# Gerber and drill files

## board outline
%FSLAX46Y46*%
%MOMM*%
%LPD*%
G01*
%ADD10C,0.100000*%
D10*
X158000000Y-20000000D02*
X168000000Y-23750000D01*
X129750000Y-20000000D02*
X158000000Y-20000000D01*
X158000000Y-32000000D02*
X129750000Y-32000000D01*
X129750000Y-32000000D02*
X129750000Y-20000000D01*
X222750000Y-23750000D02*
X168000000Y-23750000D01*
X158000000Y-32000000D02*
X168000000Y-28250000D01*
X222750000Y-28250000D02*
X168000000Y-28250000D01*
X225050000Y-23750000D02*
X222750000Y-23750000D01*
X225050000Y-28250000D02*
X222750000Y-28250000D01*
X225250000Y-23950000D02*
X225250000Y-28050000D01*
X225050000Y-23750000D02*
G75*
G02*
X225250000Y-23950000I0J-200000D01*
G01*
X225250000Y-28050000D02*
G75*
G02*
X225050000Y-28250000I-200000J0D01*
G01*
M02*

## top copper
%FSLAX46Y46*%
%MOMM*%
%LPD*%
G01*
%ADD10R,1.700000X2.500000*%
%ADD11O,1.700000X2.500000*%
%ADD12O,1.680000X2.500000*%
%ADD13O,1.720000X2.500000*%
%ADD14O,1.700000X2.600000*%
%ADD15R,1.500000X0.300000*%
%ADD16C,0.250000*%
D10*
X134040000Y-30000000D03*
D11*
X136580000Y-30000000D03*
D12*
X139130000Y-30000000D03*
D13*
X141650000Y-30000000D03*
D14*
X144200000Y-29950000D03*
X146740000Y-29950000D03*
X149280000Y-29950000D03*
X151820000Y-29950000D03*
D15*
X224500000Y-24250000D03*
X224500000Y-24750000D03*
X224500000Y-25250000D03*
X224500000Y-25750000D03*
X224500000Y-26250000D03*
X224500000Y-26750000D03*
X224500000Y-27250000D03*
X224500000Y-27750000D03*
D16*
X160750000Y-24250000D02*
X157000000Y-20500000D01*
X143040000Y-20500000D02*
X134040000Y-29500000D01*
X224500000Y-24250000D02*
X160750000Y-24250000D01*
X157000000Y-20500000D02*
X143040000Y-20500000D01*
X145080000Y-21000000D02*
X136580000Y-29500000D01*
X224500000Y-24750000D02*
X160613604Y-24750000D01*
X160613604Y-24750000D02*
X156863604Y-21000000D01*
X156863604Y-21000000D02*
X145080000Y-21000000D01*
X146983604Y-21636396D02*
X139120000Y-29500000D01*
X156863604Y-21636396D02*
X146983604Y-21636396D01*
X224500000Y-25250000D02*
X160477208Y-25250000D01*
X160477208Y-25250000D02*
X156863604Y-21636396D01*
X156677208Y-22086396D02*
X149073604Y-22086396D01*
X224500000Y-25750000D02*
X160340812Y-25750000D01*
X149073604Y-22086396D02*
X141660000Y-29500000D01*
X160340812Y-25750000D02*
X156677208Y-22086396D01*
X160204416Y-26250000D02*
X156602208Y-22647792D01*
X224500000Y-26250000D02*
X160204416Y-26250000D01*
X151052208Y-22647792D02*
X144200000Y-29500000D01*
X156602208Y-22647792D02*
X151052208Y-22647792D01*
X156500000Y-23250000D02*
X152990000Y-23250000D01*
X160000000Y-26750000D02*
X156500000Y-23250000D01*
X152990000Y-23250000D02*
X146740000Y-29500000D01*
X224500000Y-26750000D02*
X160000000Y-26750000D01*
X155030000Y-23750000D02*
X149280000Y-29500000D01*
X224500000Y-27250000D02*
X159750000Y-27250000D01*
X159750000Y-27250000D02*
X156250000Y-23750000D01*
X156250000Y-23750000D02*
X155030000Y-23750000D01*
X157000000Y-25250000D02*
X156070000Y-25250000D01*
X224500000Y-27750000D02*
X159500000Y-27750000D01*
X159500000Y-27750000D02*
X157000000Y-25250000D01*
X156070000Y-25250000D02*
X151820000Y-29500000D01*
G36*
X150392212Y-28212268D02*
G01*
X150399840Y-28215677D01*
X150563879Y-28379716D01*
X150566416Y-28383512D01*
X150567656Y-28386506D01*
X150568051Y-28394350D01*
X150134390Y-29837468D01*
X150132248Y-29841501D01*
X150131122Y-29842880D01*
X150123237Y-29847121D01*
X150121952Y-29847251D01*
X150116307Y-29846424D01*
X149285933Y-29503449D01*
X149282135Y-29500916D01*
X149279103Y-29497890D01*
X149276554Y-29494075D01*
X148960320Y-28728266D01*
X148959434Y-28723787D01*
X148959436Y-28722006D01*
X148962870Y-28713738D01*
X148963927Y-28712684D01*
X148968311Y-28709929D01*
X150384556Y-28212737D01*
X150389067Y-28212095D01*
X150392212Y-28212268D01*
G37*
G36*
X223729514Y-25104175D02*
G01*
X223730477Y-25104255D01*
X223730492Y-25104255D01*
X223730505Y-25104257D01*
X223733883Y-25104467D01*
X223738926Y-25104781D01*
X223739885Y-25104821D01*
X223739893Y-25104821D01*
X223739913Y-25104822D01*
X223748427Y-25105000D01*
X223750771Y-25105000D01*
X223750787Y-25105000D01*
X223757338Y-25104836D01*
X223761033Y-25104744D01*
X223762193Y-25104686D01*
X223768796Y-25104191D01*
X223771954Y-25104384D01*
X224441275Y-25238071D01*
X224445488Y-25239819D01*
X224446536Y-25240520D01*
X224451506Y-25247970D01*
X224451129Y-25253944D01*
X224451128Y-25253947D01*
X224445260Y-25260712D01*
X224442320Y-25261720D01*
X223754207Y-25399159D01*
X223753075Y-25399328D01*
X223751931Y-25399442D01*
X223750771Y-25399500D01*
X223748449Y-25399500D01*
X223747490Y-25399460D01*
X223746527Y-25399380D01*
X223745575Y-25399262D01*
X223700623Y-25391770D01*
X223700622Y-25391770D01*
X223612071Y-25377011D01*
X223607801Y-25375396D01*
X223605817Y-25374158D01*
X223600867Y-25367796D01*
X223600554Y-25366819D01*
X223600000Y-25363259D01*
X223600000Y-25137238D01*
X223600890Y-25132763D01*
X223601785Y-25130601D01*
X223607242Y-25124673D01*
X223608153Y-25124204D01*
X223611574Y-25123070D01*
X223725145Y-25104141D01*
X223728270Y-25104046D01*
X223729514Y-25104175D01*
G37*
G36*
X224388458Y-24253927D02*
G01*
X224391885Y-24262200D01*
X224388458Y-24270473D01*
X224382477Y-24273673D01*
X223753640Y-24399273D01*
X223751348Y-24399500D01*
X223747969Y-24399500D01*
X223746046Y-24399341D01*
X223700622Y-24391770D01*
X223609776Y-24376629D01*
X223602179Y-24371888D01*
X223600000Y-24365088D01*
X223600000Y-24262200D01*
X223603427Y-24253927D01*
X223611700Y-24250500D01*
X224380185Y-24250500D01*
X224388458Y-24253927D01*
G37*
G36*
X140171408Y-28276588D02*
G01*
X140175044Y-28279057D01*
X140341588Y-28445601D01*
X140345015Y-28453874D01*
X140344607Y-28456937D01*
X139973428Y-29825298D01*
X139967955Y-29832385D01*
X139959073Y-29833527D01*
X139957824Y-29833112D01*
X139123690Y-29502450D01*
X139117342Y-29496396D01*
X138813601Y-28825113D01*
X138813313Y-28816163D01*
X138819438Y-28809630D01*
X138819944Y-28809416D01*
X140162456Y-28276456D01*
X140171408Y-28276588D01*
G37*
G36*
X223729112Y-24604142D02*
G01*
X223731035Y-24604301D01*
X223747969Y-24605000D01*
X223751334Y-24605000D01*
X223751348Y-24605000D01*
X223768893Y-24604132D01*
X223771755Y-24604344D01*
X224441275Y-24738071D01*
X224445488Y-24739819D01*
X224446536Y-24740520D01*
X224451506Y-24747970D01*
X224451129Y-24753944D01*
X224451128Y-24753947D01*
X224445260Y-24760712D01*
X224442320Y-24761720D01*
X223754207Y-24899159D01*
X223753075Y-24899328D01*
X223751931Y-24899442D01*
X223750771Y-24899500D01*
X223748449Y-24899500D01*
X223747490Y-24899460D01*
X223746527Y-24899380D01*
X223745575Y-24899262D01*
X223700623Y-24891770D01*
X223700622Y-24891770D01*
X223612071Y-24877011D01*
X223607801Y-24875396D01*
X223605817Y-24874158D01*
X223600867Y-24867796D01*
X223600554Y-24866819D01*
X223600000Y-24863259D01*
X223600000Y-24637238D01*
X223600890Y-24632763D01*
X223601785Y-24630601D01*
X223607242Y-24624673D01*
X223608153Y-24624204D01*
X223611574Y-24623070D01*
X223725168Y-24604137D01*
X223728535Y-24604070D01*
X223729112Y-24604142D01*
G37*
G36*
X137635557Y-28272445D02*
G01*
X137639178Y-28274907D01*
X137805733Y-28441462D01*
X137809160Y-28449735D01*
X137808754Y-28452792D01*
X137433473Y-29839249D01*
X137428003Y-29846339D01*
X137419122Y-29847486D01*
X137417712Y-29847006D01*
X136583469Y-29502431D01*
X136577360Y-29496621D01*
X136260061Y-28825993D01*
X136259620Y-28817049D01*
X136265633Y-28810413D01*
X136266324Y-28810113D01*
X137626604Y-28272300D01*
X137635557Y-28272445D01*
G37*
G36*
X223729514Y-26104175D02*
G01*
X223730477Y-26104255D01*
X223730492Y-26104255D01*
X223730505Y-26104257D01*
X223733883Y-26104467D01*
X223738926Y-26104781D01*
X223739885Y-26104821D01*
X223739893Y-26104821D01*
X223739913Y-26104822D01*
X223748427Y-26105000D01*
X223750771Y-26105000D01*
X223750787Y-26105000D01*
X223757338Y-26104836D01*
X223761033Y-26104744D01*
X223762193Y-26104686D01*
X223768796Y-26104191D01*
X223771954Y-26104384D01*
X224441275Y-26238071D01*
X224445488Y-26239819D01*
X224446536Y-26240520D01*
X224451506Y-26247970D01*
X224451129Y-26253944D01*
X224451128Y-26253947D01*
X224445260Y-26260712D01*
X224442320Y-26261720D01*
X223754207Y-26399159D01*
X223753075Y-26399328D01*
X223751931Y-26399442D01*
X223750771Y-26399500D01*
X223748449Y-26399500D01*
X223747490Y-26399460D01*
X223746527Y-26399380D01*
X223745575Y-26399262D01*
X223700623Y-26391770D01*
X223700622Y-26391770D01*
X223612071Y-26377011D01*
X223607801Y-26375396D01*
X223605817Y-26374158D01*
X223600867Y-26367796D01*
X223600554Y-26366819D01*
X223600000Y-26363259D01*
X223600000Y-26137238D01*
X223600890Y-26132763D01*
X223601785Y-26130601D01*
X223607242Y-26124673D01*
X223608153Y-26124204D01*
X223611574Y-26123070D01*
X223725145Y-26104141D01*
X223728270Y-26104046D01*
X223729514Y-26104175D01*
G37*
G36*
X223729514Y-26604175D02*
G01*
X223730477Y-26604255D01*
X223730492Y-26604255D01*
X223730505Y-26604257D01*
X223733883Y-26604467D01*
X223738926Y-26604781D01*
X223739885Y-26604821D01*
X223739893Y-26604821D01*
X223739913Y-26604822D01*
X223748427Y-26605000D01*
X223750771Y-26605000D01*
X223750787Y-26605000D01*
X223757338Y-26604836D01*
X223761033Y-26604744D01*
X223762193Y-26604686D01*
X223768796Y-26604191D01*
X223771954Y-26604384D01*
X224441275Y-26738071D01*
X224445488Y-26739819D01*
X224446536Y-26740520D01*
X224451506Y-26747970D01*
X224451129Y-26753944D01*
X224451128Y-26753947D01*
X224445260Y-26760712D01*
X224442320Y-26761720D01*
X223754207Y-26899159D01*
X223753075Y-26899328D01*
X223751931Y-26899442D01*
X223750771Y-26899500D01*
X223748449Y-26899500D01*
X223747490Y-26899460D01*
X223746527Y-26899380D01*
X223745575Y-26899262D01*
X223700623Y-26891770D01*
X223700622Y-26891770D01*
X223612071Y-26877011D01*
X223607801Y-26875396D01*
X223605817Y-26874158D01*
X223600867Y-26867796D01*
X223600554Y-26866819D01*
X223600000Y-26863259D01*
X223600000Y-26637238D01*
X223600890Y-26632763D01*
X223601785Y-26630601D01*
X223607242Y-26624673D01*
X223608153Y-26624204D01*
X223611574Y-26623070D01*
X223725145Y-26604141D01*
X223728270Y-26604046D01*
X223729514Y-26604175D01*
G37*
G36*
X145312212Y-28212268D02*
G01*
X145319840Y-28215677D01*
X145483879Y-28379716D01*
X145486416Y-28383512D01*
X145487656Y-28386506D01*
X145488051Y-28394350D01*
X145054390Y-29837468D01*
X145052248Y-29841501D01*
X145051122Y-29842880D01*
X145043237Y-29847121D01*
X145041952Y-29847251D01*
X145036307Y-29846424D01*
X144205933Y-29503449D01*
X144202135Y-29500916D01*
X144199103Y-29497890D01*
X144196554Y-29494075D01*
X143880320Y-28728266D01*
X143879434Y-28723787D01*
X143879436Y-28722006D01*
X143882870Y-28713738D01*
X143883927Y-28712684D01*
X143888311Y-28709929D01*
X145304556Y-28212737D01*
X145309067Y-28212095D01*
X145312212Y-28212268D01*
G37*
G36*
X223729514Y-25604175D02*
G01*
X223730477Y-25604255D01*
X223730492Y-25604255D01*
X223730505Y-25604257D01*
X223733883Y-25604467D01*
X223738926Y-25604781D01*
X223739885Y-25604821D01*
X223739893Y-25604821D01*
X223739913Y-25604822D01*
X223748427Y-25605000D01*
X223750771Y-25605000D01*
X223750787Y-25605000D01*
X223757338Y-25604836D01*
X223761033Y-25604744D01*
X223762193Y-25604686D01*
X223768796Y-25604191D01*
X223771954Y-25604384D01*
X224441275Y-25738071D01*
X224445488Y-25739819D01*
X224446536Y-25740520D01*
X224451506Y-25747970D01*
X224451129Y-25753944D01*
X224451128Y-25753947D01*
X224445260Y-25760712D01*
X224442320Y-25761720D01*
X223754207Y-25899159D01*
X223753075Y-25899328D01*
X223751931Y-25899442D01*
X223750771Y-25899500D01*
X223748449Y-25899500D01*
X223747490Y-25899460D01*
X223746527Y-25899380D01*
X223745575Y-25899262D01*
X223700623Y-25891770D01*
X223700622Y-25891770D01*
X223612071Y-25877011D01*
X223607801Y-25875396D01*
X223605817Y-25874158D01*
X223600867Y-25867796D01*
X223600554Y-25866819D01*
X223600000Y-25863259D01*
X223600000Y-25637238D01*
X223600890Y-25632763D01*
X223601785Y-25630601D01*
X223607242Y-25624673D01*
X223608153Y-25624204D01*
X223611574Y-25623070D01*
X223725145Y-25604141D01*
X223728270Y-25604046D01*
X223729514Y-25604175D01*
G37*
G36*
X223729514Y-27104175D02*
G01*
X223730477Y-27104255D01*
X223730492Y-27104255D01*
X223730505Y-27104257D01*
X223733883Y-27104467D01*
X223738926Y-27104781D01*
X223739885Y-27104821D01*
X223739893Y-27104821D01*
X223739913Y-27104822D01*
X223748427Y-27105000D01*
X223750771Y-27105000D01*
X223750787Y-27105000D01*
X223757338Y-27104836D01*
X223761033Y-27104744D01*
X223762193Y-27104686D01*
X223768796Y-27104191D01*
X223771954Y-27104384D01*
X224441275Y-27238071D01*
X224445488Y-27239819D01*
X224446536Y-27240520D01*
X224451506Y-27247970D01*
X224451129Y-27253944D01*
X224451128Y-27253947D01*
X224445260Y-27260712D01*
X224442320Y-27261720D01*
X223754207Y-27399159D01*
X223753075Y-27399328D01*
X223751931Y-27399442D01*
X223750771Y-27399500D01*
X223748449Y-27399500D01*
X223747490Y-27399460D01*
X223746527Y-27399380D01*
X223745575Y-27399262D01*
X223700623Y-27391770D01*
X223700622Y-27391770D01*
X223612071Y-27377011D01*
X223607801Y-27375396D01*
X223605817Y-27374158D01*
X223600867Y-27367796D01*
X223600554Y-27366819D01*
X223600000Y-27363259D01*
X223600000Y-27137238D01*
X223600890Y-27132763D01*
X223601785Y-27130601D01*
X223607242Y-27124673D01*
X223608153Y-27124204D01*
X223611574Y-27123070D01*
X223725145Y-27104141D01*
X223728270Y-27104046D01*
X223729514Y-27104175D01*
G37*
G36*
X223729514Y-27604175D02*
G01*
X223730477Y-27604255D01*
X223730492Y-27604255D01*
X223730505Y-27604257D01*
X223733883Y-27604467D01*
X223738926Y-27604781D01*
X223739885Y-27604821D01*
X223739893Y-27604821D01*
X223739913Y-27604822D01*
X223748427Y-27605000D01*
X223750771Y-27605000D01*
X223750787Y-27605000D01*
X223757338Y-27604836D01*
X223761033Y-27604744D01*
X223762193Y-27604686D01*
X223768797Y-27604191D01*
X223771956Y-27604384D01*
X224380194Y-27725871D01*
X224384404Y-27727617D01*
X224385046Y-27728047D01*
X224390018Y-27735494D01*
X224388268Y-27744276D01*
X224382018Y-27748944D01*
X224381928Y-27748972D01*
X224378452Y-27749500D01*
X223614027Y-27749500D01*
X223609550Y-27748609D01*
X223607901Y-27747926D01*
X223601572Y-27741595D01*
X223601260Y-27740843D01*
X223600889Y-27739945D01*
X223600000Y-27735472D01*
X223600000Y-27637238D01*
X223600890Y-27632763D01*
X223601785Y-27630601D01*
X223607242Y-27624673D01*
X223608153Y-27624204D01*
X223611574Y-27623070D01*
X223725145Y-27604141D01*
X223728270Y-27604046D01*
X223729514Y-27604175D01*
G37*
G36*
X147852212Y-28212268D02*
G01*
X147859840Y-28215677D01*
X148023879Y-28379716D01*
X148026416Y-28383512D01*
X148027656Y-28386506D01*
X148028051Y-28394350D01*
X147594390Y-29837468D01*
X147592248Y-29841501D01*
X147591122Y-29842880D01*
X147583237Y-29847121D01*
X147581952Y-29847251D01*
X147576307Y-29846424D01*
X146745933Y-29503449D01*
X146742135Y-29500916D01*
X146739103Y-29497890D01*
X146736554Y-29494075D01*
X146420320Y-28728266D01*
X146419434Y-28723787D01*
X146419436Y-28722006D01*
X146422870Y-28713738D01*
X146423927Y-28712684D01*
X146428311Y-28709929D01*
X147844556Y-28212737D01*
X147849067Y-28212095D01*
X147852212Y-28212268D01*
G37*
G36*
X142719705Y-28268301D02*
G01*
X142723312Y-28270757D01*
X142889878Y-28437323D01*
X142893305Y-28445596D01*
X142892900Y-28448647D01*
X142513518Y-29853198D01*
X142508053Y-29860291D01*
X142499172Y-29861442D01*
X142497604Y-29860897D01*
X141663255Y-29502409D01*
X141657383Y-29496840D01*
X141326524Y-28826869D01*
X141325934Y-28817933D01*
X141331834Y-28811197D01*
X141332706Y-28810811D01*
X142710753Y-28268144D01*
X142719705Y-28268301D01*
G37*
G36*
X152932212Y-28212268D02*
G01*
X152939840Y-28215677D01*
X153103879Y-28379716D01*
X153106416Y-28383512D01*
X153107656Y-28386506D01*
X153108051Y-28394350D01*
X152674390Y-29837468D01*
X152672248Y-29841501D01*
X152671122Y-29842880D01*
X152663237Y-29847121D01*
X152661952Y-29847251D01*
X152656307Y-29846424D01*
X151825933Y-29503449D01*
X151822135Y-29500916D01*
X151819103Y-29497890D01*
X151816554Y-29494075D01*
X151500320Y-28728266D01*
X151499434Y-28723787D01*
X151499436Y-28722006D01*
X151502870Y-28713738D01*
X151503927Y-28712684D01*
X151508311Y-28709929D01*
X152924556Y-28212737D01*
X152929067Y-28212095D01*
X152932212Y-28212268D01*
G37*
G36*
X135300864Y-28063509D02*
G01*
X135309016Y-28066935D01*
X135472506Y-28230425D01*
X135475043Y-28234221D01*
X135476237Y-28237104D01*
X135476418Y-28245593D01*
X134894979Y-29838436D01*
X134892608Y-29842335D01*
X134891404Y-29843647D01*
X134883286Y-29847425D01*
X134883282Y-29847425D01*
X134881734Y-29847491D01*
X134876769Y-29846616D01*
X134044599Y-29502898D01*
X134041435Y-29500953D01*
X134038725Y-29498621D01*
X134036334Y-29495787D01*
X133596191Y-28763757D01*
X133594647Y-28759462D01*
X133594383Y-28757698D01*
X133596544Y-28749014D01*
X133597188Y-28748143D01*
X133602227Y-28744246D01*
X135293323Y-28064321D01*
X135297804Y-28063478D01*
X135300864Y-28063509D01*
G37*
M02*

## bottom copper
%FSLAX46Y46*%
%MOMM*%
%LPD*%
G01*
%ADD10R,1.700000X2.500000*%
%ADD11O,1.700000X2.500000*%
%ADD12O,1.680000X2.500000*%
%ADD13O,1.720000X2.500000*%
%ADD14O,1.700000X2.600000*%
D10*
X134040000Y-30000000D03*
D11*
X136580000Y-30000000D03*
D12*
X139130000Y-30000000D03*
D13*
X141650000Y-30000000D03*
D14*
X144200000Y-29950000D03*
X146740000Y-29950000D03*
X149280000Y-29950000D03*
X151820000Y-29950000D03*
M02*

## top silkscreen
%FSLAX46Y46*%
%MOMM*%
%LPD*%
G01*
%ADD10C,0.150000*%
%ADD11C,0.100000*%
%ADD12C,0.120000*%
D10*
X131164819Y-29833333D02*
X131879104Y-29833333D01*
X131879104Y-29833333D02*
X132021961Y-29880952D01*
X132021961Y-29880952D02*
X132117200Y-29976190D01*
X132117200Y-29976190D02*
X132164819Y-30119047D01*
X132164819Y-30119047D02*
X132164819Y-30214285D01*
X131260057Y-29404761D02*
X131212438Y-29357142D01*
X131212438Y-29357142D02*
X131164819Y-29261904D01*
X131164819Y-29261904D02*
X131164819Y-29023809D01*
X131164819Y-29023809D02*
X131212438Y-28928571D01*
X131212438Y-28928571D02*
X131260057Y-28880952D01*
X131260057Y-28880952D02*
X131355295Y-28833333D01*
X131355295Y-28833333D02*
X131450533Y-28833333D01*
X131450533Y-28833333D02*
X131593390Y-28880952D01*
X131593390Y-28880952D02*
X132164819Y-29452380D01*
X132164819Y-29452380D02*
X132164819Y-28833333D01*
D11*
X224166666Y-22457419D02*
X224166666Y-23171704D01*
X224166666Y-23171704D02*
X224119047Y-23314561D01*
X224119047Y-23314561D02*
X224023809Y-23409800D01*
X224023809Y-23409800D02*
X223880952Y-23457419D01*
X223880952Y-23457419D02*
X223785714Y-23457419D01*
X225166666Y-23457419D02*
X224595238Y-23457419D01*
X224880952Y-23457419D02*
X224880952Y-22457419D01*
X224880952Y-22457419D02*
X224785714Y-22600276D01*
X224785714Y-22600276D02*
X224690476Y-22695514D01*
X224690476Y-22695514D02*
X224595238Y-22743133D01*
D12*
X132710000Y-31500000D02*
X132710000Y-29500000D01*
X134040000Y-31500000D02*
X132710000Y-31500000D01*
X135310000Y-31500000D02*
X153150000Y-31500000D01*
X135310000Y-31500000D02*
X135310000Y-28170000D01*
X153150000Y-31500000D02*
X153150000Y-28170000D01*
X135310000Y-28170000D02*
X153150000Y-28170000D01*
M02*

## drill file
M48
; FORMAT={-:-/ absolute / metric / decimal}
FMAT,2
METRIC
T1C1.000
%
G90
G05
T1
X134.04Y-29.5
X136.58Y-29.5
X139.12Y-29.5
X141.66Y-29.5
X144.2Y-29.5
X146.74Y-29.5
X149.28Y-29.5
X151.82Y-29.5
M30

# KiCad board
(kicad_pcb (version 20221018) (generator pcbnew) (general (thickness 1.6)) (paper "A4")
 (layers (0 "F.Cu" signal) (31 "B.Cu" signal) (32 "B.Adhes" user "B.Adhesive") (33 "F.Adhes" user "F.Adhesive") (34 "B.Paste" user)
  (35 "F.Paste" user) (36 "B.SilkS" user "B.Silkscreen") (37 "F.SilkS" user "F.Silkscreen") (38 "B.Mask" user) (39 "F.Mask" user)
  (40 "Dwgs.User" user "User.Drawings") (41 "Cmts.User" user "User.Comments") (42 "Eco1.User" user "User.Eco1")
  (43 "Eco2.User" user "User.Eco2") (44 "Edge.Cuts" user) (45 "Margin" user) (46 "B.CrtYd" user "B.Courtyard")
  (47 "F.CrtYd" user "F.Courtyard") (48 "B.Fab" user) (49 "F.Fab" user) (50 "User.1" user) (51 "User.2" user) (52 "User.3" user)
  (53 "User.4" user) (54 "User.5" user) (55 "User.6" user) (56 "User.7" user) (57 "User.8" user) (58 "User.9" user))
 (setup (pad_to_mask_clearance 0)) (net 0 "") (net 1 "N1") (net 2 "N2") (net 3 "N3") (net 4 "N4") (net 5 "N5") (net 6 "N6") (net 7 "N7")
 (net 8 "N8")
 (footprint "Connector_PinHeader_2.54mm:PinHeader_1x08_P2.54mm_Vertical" (layer "F.Cu") (at 134.04 29.5 90)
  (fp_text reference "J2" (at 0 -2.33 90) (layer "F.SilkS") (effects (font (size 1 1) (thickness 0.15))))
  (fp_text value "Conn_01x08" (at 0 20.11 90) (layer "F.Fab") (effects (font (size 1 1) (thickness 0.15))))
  (fp_line (start -2 -1.33) (end 0 -1.33) (stroke (width 0.12) (type solid)) (layer "F.SilkS"))
  (fp_line (start -2 0) (end -2 -1.33) (stroke (width 0.12) (type solid)) (layer "F.SilkS"))
  (fp_line (start -2 1.27) (end -2 19.11) (stroke (width 0.12) (type solid)) (layer "F.SilkS"))
  (fp_line (start -2 1.27) (end 1.33 1.27) (stroke (width 0.12) (type solid)) (layer "F.SilkS"))
  (fp_line (start -2 19.11) (end 1.33 19.11) (stroke (width 0.12) (type solid)) (layer "F.SilkS"))
  (fp_line (start 1.33 1.27) (end 1.33 19.11) (stroke (width 0.12) (type solid)) (layer "F.SilkS"))
  (pad "1" thru_hole rect (at 0 0 90) (size 2.5 1.7) (drill 1 (offset -0.5 0)) (layers "*.Cu" "*.Mask") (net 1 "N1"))
  (pad "2" thru_hole oval (at 0 2.54 90) (size 2.5 1.7) (drill 1 (offset -0.5 0)) (layers "*.Cu" "*.Mask") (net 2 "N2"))
  (pad "3" thru_hole oval (at 0 5.08 90) (size 2.5 1.68) (drill 1 (offset -0.5 0.01)) (layers "*.Cu" "*.Mask") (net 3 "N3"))
  (pad "4" thru_hole oval (at 0 7.62 90) (size 2.5 1.72) (drill 1 (offset -0.5 -0.01)) (layers "*.Cu" "*.Mask") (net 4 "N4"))
  (pad "5" thru_hole oval (at 0 10.16 90) (size 2.6 1.7) (drill 1 (offset -0.45 0)) (layers "*.Cu" "*.Mask") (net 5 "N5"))
  (pad "6" thru_hole oval (at 0 12.7 90) (size 2.6 1.7) (drill 1 (offset -0.45 0)) (layers "*.Cu" "*.Mask") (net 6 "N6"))
  (pad "7" thru_hole oval (at 0 15.24 90) (size 2.6 1.7) (drill 1 (offset -0.45 0)) (layers "*.Cu" "*.Mask") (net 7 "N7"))
  (pad "8" thru_hole oval (at 0 17.78 90) (size 2.6 1.7) (drill 1 (offset -0.45 0)) (layers "*.Cu" "*.Mask") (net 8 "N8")))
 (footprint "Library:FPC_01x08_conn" (layer "F.Cu") (at 224.5 26)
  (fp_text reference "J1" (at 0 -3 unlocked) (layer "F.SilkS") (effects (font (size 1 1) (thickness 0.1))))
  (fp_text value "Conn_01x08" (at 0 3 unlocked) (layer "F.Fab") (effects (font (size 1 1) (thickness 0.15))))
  (fp_line (start 0.55 -2.25) (end -1.75 -2.25) (stroke (width 0.1) (type default)) (layer "Edge.Cuts"))
  (fp_line (start 0.55 2.25) (end -1.75 2.25) (stroke (width 0.1) (type default)) (layer "Edge.Cuts"))
  (fp_line (start 0.75 -2.05) (end 0.75 2.05) (stroke (width 0.1) (type default)) (layer "Edge.Cuts"))
  (fp_arc (start 0.55 -2.25) (mid 0.691422 -2.191422) (end 0.75 -2.05) (stroke (width 0.1) (type default)) (layer "Edge.Cuts"))
  (fp_arc (start 0.75 2.05) (mid 0.691422 2.191422) (end 0.55 2.25) (stroke (width 0.1) (type default)) (layer "Edge.Cuts"))
  (pad "1" smd rect (at 0 -1.75) (size 1.5 0.3) (layers "F.Cu" "F.Paste" "F.Mask") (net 1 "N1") (thermal_bridge_angle 45))
  (pad "2" smd rect (at 0 -1.25) (size 1.5 0.3) (layers "F.Cu" "F.Paste" "F.Mask") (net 2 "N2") (thermal_bridge_angle 45))
  (pad "3" smd rect (at 0 -0.75) (size 1.5 0.3) (layers "F.Cu" "F.Paste" "F.Mask") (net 3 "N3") (thermal_bridge_angle 45))
  (pad "4" smd rect (at 0 -0.25) (size 1.5 0.3) (layers "F.Cu" "F.Paste" "F.Mask") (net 4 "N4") (thermal_bridge_angle 45))
  (pad "5" smd rect (at 0 0.25) (size 1.5 0.3) (layers "F.Cu" "F.Paste" "F.Mask") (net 5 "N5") (thermal_bridge_angle 45))
  (pad "6" smd rect (at 0 0.75) (size 1.5 0.3) (layers "F.Cu" "F.Paste" "F.Mask") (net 6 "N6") (thermal_bridge_angle 45))
  (pad "7" smd rect (at 0 1.25) (size 1.5 0.3) (layers "F.Cu" "F.Paste" "F.Mask") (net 7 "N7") (thermal_bridge_angle 45))
  (pad "8" smd rect (at 0 1.75) (size 1.5 0.3) (layers "F.Cu" "F.Paste" "F.Mask") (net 8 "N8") (thermal_bridge_angle 45)))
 (gr_line (start 158 20) (end 168 23.75) (stroke (width 0.1) (type default)) (layer "Edge.Cuts"))
 (gr_line (start 129.75 20) (end 158 20) (stroke (width 0.1) (type default)) (layer "Edge.Cuts"))
 (gr_line (start 158 32) (end 129.75 32) (stroke (width 0.1) (type default)) (layer "Edge.Cuts"))
 (gr_line (start 129.75 32) (end 129.75 20) (stroke (width 0.1) (type default)) (layer "Edge.Cuts"))
 (gr_line (start 222.75 23.75) (end 168 23.75) (stroke (width 0.1) (type default)) (layer "Edge.Cuts"))
 (gr_line (start 158 32) (end 168 28.25) (stroke (width 0.1) (type default)) (layer "Edge.Cuts"))
 (gr_line (start 222.75 28.25) (end 168 28.25) (stroke (width 0.1) (type default)) (layer "Edge.Cuts"))
 (segment (start 160.75 24.25) (end 157 20.5) (width 0.25) (layer "F.Cu") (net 1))
 (segment (start 143.04 20.5) (end 134.04 29.5) (width 0.25) (layer "F.Cu") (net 1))
 (segment (start 224.5 24.25) (end 160.75 24.25) (width 0.25) (layer "F.Cu") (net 1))
 (segment (start 157 20.5) (end 143.04 20.5) (width 0.25) (layer "F.Cu") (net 1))
 (segment (start 145.08 21) (end 136.58 29.5) (width 0.25) (layer "F.Cu") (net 2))
 (segment (start 224.5 24.75) (end 160.613604 24.75) (width 0.25) (layer "F.Cu") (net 2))
 (segment (start 160.613604 24.75) (end 156.863604 21) (width 0.25) (layer "F.Cu") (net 2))
 (segment (start 156.863604 21) (end 145.08 21) (width 0.25) (layer "F.Cu") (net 2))
 (segment (start 146.983604 21.636396) (end 139.12 29.5) (width 0.25) (layer "F.Cu") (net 3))
 (segment (start 156.863604 21.636396) (end 146.983604 21.636396) (width 0.25) (layer "F.Cu") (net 3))
 (segment (start 224.5 25.25) (end 160.477208 25.25) (width 0.25) (layer "F.Cu") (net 3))
 (segment (start 160.477208 25.25) (end 156.863604 21.636396) (width 0.25) (layer "F.Cu") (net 3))
 (segment (start 156.677208 22.086396) (end 149.073604 22.086396) (width 0.25) (layer "F.Cu") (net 4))
 (segment (start 224.5 25.75) (end 160.340812 25.75) (width 0.25) (layer "F.Cu") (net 4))
 (segment (start 149.073604 22.086396) (end 141.66 29.5) (width 0.25) (layer "F.Cu") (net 4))
 (segment (start 160.340812 25.75) (end 156.677208 22.086396) (width 0.25) (layer "F.Cu") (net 4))
 (segment (start 160.204416 26.25) (end 156.602208 22.647792) (width 0.25) (layer "F.Cu") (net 5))
 (segment (start 224.5 26.25) (end 160.204416 26.25) (width 0.25) (layer "F.Cu") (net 5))
 (segment (start 151.052208 22.647792) (end 144.2 29.5) (width 0.25) (layer "F.Cu") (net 5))
 (segment (start 156.602208 22.647792) (end 151.052208 22.647792) (width 0.25) (layer "F.Cu") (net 5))
 (segment (start 156.5 23.25) (end 152.99 23.25) (width 0.25) (layer "F.Cu") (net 6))
 (segment (start 160 26.75) (end 156.5 23.25) (width 0.25) (layer "F.Cu") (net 6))
 (segment (start 152.99 23.25) (end 146.74 29.5) (width 0.25) (layer "F.Cu") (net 6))
 (segment (start 224.5 26.75) (end 160 26.75) (width 0.25) (layer "F.Cu") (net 6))
 (segment (start 155.03 23.75) (end 149.28 29.5) (width 0.25) (layer "F.Cu") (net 7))
 (segment (start 224.5 27.25) (end 159.75 27.25) (width 0.25) (layer "F.Cu") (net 7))
 (segment (start 159.75 27.25) (end 156.25 23.75) (width 0.25) (layer "F.Cu") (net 7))
 (segment (start 156.25 23.75) (end 155.03 23.75) (width 0.25) (layer "F.Cu") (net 7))
 (segment (start 157 25.25) (end 156.07 25.25) (width 0.25) (layer "F.Cu") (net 8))
 (segment (start 224.5 27.75) (end 159.5 27.75) (width 0.25) (layer "F.Cu") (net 8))
 (segment (start 159.5 27.75) (end 157 25.25) (width 0.25) (layer "F.Cu") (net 8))
 (segment (start 156.07 25.25) (end 151.82 29.5) (width 0.25) (layer "F.Cu") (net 8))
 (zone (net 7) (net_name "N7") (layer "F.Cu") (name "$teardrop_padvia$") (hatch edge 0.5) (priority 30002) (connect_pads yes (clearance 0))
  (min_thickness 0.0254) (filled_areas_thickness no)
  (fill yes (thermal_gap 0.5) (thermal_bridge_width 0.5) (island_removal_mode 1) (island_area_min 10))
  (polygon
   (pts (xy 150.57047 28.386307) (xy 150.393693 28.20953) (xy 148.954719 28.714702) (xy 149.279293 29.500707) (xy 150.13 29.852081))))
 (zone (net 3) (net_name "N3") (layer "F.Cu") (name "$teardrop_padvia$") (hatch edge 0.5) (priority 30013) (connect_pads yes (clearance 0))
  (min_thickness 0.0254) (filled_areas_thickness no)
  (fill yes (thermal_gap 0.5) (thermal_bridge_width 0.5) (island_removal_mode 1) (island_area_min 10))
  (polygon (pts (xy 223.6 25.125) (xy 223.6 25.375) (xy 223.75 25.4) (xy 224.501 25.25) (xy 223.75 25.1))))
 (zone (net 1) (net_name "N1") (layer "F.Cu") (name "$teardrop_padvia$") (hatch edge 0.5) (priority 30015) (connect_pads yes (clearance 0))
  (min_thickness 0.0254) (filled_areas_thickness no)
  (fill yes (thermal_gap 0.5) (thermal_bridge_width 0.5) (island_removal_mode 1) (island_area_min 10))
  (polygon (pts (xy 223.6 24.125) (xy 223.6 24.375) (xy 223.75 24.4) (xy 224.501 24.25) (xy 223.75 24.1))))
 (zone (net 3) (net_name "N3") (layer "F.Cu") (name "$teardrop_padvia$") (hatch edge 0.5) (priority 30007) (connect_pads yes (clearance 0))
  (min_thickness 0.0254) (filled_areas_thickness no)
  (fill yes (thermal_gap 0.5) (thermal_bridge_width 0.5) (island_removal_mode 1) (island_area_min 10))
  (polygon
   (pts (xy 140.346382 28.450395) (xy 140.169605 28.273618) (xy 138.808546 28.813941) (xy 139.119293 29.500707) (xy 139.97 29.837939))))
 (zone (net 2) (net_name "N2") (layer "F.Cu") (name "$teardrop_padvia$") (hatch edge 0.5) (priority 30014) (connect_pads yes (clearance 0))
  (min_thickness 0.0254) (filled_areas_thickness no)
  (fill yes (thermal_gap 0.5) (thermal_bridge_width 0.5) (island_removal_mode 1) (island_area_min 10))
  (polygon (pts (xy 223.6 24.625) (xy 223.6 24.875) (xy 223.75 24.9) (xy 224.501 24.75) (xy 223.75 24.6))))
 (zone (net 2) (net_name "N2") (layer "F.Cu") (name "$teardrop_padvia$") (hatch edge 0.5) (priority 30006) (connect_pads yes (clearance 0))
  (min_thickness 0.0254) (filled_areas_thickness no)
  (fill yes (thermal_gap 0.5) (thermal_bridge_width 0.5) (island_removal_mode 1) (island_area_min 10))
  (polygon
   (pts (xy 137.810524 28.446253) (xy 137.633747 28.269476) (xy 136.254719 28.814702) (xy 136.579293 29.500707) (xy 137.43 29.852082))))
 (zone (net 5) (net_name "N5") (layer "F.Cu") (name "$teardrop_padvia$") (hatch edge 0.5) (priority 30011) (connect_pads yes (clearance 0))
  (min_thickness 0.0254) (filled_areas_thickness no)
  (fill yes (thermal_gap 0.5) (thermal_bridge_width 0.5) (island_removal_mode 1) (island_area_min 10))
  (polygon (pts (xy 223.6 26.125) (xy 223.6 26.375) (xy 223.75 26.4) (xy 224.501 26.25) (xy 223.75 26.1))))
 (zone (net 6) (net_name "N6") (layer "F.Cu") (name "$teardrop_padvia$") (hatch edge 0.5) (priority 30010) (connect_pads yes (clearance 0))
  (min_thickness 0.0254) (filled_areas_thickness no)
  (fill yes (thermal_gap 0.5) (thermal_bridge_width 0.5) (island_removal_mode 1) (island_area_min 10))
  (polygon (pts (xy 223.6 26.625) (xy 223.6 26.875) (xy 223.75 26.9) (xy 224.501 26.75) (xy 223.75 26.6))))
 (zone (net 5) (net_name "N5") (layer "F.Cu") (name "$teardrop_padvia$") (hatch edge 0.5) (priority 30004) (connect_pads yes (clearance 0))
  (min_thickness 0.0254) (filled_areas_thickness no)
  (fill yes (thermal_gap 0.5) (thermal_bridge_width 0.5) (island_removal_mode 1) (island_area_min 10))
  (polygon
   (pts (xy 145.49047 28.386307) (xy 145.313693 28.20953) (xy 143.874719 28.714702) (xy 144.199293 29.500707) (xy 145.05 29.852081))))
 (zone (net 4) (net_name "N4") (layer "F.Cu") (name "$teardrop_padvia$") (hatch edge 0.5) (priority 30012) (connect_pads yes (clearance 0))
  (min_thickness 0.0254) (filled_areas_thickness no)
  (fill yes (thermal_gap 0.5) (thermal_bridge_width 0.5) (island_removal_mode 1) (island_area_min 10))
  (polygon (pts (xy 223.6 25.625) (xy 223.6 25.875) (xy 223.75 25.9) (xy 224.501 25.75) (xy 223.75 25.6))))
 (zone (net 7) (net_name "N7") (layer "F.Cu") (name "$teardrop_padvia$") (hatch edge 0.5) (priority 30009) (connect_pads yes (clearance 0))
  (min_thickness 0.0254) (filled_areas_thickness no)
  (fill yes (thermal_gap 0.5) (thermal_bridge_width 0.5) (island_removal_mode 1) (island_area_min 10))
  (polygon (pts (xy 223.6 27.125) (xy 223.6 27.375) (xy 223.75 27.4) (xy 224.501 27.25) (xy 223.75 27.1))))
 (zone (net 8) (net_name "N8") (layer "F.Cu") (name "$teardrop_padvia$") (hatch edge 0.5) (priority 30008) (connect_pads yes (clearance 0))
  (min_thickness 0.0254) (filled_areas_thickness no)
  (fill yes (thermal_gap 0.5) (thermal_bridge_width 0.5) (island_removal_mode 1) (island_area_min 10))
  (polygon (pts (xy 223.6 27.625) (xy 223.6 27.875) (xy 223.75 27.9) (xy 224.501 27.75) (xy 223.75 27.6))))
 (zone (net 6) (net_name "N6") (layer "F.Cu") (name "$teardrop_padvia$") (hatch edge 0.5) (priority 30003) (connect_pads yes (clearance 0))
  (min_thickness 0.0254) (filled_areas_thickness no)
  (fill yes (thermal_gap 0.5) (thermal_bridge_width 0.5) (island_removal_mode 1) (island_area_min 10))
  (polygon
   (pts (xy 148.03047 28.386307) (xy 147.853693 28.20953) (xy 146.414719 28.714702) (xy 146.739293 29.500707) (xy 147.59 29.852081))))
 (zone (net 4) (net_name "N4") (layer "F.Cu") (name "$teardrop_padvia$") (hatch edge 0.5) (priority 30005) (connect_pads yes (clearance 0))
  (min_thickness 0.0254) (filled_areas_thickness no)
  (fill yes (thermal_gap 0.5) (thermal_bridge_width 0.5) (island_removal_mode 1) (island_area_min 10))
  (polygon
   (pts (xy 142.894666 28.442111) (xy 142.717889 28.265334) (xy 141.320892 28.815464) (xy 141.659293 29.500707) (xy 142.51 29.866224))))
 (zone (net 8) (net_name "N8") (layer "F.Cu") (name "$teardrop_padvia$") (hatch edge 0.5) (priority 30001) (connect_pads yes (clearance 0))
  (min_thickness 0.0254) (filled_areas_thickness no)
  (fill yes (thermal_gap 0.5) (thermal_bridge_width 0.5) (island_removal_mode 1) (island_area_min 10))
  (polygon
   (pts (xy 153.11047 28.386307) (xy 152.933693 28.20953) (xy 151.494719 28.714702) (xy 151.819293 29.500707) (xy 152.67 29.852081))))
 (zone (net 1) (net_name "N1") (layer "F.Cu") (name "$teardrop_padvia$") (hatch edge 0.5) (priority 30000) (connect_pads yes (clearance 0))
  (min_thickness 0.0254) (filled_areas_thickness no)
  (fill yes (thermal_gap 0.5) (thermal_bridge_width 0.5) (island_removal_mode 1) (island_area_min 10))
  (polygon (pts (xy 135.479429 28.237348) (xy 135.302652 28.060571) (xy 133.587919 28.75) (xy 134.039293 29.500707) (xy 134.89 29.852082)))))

